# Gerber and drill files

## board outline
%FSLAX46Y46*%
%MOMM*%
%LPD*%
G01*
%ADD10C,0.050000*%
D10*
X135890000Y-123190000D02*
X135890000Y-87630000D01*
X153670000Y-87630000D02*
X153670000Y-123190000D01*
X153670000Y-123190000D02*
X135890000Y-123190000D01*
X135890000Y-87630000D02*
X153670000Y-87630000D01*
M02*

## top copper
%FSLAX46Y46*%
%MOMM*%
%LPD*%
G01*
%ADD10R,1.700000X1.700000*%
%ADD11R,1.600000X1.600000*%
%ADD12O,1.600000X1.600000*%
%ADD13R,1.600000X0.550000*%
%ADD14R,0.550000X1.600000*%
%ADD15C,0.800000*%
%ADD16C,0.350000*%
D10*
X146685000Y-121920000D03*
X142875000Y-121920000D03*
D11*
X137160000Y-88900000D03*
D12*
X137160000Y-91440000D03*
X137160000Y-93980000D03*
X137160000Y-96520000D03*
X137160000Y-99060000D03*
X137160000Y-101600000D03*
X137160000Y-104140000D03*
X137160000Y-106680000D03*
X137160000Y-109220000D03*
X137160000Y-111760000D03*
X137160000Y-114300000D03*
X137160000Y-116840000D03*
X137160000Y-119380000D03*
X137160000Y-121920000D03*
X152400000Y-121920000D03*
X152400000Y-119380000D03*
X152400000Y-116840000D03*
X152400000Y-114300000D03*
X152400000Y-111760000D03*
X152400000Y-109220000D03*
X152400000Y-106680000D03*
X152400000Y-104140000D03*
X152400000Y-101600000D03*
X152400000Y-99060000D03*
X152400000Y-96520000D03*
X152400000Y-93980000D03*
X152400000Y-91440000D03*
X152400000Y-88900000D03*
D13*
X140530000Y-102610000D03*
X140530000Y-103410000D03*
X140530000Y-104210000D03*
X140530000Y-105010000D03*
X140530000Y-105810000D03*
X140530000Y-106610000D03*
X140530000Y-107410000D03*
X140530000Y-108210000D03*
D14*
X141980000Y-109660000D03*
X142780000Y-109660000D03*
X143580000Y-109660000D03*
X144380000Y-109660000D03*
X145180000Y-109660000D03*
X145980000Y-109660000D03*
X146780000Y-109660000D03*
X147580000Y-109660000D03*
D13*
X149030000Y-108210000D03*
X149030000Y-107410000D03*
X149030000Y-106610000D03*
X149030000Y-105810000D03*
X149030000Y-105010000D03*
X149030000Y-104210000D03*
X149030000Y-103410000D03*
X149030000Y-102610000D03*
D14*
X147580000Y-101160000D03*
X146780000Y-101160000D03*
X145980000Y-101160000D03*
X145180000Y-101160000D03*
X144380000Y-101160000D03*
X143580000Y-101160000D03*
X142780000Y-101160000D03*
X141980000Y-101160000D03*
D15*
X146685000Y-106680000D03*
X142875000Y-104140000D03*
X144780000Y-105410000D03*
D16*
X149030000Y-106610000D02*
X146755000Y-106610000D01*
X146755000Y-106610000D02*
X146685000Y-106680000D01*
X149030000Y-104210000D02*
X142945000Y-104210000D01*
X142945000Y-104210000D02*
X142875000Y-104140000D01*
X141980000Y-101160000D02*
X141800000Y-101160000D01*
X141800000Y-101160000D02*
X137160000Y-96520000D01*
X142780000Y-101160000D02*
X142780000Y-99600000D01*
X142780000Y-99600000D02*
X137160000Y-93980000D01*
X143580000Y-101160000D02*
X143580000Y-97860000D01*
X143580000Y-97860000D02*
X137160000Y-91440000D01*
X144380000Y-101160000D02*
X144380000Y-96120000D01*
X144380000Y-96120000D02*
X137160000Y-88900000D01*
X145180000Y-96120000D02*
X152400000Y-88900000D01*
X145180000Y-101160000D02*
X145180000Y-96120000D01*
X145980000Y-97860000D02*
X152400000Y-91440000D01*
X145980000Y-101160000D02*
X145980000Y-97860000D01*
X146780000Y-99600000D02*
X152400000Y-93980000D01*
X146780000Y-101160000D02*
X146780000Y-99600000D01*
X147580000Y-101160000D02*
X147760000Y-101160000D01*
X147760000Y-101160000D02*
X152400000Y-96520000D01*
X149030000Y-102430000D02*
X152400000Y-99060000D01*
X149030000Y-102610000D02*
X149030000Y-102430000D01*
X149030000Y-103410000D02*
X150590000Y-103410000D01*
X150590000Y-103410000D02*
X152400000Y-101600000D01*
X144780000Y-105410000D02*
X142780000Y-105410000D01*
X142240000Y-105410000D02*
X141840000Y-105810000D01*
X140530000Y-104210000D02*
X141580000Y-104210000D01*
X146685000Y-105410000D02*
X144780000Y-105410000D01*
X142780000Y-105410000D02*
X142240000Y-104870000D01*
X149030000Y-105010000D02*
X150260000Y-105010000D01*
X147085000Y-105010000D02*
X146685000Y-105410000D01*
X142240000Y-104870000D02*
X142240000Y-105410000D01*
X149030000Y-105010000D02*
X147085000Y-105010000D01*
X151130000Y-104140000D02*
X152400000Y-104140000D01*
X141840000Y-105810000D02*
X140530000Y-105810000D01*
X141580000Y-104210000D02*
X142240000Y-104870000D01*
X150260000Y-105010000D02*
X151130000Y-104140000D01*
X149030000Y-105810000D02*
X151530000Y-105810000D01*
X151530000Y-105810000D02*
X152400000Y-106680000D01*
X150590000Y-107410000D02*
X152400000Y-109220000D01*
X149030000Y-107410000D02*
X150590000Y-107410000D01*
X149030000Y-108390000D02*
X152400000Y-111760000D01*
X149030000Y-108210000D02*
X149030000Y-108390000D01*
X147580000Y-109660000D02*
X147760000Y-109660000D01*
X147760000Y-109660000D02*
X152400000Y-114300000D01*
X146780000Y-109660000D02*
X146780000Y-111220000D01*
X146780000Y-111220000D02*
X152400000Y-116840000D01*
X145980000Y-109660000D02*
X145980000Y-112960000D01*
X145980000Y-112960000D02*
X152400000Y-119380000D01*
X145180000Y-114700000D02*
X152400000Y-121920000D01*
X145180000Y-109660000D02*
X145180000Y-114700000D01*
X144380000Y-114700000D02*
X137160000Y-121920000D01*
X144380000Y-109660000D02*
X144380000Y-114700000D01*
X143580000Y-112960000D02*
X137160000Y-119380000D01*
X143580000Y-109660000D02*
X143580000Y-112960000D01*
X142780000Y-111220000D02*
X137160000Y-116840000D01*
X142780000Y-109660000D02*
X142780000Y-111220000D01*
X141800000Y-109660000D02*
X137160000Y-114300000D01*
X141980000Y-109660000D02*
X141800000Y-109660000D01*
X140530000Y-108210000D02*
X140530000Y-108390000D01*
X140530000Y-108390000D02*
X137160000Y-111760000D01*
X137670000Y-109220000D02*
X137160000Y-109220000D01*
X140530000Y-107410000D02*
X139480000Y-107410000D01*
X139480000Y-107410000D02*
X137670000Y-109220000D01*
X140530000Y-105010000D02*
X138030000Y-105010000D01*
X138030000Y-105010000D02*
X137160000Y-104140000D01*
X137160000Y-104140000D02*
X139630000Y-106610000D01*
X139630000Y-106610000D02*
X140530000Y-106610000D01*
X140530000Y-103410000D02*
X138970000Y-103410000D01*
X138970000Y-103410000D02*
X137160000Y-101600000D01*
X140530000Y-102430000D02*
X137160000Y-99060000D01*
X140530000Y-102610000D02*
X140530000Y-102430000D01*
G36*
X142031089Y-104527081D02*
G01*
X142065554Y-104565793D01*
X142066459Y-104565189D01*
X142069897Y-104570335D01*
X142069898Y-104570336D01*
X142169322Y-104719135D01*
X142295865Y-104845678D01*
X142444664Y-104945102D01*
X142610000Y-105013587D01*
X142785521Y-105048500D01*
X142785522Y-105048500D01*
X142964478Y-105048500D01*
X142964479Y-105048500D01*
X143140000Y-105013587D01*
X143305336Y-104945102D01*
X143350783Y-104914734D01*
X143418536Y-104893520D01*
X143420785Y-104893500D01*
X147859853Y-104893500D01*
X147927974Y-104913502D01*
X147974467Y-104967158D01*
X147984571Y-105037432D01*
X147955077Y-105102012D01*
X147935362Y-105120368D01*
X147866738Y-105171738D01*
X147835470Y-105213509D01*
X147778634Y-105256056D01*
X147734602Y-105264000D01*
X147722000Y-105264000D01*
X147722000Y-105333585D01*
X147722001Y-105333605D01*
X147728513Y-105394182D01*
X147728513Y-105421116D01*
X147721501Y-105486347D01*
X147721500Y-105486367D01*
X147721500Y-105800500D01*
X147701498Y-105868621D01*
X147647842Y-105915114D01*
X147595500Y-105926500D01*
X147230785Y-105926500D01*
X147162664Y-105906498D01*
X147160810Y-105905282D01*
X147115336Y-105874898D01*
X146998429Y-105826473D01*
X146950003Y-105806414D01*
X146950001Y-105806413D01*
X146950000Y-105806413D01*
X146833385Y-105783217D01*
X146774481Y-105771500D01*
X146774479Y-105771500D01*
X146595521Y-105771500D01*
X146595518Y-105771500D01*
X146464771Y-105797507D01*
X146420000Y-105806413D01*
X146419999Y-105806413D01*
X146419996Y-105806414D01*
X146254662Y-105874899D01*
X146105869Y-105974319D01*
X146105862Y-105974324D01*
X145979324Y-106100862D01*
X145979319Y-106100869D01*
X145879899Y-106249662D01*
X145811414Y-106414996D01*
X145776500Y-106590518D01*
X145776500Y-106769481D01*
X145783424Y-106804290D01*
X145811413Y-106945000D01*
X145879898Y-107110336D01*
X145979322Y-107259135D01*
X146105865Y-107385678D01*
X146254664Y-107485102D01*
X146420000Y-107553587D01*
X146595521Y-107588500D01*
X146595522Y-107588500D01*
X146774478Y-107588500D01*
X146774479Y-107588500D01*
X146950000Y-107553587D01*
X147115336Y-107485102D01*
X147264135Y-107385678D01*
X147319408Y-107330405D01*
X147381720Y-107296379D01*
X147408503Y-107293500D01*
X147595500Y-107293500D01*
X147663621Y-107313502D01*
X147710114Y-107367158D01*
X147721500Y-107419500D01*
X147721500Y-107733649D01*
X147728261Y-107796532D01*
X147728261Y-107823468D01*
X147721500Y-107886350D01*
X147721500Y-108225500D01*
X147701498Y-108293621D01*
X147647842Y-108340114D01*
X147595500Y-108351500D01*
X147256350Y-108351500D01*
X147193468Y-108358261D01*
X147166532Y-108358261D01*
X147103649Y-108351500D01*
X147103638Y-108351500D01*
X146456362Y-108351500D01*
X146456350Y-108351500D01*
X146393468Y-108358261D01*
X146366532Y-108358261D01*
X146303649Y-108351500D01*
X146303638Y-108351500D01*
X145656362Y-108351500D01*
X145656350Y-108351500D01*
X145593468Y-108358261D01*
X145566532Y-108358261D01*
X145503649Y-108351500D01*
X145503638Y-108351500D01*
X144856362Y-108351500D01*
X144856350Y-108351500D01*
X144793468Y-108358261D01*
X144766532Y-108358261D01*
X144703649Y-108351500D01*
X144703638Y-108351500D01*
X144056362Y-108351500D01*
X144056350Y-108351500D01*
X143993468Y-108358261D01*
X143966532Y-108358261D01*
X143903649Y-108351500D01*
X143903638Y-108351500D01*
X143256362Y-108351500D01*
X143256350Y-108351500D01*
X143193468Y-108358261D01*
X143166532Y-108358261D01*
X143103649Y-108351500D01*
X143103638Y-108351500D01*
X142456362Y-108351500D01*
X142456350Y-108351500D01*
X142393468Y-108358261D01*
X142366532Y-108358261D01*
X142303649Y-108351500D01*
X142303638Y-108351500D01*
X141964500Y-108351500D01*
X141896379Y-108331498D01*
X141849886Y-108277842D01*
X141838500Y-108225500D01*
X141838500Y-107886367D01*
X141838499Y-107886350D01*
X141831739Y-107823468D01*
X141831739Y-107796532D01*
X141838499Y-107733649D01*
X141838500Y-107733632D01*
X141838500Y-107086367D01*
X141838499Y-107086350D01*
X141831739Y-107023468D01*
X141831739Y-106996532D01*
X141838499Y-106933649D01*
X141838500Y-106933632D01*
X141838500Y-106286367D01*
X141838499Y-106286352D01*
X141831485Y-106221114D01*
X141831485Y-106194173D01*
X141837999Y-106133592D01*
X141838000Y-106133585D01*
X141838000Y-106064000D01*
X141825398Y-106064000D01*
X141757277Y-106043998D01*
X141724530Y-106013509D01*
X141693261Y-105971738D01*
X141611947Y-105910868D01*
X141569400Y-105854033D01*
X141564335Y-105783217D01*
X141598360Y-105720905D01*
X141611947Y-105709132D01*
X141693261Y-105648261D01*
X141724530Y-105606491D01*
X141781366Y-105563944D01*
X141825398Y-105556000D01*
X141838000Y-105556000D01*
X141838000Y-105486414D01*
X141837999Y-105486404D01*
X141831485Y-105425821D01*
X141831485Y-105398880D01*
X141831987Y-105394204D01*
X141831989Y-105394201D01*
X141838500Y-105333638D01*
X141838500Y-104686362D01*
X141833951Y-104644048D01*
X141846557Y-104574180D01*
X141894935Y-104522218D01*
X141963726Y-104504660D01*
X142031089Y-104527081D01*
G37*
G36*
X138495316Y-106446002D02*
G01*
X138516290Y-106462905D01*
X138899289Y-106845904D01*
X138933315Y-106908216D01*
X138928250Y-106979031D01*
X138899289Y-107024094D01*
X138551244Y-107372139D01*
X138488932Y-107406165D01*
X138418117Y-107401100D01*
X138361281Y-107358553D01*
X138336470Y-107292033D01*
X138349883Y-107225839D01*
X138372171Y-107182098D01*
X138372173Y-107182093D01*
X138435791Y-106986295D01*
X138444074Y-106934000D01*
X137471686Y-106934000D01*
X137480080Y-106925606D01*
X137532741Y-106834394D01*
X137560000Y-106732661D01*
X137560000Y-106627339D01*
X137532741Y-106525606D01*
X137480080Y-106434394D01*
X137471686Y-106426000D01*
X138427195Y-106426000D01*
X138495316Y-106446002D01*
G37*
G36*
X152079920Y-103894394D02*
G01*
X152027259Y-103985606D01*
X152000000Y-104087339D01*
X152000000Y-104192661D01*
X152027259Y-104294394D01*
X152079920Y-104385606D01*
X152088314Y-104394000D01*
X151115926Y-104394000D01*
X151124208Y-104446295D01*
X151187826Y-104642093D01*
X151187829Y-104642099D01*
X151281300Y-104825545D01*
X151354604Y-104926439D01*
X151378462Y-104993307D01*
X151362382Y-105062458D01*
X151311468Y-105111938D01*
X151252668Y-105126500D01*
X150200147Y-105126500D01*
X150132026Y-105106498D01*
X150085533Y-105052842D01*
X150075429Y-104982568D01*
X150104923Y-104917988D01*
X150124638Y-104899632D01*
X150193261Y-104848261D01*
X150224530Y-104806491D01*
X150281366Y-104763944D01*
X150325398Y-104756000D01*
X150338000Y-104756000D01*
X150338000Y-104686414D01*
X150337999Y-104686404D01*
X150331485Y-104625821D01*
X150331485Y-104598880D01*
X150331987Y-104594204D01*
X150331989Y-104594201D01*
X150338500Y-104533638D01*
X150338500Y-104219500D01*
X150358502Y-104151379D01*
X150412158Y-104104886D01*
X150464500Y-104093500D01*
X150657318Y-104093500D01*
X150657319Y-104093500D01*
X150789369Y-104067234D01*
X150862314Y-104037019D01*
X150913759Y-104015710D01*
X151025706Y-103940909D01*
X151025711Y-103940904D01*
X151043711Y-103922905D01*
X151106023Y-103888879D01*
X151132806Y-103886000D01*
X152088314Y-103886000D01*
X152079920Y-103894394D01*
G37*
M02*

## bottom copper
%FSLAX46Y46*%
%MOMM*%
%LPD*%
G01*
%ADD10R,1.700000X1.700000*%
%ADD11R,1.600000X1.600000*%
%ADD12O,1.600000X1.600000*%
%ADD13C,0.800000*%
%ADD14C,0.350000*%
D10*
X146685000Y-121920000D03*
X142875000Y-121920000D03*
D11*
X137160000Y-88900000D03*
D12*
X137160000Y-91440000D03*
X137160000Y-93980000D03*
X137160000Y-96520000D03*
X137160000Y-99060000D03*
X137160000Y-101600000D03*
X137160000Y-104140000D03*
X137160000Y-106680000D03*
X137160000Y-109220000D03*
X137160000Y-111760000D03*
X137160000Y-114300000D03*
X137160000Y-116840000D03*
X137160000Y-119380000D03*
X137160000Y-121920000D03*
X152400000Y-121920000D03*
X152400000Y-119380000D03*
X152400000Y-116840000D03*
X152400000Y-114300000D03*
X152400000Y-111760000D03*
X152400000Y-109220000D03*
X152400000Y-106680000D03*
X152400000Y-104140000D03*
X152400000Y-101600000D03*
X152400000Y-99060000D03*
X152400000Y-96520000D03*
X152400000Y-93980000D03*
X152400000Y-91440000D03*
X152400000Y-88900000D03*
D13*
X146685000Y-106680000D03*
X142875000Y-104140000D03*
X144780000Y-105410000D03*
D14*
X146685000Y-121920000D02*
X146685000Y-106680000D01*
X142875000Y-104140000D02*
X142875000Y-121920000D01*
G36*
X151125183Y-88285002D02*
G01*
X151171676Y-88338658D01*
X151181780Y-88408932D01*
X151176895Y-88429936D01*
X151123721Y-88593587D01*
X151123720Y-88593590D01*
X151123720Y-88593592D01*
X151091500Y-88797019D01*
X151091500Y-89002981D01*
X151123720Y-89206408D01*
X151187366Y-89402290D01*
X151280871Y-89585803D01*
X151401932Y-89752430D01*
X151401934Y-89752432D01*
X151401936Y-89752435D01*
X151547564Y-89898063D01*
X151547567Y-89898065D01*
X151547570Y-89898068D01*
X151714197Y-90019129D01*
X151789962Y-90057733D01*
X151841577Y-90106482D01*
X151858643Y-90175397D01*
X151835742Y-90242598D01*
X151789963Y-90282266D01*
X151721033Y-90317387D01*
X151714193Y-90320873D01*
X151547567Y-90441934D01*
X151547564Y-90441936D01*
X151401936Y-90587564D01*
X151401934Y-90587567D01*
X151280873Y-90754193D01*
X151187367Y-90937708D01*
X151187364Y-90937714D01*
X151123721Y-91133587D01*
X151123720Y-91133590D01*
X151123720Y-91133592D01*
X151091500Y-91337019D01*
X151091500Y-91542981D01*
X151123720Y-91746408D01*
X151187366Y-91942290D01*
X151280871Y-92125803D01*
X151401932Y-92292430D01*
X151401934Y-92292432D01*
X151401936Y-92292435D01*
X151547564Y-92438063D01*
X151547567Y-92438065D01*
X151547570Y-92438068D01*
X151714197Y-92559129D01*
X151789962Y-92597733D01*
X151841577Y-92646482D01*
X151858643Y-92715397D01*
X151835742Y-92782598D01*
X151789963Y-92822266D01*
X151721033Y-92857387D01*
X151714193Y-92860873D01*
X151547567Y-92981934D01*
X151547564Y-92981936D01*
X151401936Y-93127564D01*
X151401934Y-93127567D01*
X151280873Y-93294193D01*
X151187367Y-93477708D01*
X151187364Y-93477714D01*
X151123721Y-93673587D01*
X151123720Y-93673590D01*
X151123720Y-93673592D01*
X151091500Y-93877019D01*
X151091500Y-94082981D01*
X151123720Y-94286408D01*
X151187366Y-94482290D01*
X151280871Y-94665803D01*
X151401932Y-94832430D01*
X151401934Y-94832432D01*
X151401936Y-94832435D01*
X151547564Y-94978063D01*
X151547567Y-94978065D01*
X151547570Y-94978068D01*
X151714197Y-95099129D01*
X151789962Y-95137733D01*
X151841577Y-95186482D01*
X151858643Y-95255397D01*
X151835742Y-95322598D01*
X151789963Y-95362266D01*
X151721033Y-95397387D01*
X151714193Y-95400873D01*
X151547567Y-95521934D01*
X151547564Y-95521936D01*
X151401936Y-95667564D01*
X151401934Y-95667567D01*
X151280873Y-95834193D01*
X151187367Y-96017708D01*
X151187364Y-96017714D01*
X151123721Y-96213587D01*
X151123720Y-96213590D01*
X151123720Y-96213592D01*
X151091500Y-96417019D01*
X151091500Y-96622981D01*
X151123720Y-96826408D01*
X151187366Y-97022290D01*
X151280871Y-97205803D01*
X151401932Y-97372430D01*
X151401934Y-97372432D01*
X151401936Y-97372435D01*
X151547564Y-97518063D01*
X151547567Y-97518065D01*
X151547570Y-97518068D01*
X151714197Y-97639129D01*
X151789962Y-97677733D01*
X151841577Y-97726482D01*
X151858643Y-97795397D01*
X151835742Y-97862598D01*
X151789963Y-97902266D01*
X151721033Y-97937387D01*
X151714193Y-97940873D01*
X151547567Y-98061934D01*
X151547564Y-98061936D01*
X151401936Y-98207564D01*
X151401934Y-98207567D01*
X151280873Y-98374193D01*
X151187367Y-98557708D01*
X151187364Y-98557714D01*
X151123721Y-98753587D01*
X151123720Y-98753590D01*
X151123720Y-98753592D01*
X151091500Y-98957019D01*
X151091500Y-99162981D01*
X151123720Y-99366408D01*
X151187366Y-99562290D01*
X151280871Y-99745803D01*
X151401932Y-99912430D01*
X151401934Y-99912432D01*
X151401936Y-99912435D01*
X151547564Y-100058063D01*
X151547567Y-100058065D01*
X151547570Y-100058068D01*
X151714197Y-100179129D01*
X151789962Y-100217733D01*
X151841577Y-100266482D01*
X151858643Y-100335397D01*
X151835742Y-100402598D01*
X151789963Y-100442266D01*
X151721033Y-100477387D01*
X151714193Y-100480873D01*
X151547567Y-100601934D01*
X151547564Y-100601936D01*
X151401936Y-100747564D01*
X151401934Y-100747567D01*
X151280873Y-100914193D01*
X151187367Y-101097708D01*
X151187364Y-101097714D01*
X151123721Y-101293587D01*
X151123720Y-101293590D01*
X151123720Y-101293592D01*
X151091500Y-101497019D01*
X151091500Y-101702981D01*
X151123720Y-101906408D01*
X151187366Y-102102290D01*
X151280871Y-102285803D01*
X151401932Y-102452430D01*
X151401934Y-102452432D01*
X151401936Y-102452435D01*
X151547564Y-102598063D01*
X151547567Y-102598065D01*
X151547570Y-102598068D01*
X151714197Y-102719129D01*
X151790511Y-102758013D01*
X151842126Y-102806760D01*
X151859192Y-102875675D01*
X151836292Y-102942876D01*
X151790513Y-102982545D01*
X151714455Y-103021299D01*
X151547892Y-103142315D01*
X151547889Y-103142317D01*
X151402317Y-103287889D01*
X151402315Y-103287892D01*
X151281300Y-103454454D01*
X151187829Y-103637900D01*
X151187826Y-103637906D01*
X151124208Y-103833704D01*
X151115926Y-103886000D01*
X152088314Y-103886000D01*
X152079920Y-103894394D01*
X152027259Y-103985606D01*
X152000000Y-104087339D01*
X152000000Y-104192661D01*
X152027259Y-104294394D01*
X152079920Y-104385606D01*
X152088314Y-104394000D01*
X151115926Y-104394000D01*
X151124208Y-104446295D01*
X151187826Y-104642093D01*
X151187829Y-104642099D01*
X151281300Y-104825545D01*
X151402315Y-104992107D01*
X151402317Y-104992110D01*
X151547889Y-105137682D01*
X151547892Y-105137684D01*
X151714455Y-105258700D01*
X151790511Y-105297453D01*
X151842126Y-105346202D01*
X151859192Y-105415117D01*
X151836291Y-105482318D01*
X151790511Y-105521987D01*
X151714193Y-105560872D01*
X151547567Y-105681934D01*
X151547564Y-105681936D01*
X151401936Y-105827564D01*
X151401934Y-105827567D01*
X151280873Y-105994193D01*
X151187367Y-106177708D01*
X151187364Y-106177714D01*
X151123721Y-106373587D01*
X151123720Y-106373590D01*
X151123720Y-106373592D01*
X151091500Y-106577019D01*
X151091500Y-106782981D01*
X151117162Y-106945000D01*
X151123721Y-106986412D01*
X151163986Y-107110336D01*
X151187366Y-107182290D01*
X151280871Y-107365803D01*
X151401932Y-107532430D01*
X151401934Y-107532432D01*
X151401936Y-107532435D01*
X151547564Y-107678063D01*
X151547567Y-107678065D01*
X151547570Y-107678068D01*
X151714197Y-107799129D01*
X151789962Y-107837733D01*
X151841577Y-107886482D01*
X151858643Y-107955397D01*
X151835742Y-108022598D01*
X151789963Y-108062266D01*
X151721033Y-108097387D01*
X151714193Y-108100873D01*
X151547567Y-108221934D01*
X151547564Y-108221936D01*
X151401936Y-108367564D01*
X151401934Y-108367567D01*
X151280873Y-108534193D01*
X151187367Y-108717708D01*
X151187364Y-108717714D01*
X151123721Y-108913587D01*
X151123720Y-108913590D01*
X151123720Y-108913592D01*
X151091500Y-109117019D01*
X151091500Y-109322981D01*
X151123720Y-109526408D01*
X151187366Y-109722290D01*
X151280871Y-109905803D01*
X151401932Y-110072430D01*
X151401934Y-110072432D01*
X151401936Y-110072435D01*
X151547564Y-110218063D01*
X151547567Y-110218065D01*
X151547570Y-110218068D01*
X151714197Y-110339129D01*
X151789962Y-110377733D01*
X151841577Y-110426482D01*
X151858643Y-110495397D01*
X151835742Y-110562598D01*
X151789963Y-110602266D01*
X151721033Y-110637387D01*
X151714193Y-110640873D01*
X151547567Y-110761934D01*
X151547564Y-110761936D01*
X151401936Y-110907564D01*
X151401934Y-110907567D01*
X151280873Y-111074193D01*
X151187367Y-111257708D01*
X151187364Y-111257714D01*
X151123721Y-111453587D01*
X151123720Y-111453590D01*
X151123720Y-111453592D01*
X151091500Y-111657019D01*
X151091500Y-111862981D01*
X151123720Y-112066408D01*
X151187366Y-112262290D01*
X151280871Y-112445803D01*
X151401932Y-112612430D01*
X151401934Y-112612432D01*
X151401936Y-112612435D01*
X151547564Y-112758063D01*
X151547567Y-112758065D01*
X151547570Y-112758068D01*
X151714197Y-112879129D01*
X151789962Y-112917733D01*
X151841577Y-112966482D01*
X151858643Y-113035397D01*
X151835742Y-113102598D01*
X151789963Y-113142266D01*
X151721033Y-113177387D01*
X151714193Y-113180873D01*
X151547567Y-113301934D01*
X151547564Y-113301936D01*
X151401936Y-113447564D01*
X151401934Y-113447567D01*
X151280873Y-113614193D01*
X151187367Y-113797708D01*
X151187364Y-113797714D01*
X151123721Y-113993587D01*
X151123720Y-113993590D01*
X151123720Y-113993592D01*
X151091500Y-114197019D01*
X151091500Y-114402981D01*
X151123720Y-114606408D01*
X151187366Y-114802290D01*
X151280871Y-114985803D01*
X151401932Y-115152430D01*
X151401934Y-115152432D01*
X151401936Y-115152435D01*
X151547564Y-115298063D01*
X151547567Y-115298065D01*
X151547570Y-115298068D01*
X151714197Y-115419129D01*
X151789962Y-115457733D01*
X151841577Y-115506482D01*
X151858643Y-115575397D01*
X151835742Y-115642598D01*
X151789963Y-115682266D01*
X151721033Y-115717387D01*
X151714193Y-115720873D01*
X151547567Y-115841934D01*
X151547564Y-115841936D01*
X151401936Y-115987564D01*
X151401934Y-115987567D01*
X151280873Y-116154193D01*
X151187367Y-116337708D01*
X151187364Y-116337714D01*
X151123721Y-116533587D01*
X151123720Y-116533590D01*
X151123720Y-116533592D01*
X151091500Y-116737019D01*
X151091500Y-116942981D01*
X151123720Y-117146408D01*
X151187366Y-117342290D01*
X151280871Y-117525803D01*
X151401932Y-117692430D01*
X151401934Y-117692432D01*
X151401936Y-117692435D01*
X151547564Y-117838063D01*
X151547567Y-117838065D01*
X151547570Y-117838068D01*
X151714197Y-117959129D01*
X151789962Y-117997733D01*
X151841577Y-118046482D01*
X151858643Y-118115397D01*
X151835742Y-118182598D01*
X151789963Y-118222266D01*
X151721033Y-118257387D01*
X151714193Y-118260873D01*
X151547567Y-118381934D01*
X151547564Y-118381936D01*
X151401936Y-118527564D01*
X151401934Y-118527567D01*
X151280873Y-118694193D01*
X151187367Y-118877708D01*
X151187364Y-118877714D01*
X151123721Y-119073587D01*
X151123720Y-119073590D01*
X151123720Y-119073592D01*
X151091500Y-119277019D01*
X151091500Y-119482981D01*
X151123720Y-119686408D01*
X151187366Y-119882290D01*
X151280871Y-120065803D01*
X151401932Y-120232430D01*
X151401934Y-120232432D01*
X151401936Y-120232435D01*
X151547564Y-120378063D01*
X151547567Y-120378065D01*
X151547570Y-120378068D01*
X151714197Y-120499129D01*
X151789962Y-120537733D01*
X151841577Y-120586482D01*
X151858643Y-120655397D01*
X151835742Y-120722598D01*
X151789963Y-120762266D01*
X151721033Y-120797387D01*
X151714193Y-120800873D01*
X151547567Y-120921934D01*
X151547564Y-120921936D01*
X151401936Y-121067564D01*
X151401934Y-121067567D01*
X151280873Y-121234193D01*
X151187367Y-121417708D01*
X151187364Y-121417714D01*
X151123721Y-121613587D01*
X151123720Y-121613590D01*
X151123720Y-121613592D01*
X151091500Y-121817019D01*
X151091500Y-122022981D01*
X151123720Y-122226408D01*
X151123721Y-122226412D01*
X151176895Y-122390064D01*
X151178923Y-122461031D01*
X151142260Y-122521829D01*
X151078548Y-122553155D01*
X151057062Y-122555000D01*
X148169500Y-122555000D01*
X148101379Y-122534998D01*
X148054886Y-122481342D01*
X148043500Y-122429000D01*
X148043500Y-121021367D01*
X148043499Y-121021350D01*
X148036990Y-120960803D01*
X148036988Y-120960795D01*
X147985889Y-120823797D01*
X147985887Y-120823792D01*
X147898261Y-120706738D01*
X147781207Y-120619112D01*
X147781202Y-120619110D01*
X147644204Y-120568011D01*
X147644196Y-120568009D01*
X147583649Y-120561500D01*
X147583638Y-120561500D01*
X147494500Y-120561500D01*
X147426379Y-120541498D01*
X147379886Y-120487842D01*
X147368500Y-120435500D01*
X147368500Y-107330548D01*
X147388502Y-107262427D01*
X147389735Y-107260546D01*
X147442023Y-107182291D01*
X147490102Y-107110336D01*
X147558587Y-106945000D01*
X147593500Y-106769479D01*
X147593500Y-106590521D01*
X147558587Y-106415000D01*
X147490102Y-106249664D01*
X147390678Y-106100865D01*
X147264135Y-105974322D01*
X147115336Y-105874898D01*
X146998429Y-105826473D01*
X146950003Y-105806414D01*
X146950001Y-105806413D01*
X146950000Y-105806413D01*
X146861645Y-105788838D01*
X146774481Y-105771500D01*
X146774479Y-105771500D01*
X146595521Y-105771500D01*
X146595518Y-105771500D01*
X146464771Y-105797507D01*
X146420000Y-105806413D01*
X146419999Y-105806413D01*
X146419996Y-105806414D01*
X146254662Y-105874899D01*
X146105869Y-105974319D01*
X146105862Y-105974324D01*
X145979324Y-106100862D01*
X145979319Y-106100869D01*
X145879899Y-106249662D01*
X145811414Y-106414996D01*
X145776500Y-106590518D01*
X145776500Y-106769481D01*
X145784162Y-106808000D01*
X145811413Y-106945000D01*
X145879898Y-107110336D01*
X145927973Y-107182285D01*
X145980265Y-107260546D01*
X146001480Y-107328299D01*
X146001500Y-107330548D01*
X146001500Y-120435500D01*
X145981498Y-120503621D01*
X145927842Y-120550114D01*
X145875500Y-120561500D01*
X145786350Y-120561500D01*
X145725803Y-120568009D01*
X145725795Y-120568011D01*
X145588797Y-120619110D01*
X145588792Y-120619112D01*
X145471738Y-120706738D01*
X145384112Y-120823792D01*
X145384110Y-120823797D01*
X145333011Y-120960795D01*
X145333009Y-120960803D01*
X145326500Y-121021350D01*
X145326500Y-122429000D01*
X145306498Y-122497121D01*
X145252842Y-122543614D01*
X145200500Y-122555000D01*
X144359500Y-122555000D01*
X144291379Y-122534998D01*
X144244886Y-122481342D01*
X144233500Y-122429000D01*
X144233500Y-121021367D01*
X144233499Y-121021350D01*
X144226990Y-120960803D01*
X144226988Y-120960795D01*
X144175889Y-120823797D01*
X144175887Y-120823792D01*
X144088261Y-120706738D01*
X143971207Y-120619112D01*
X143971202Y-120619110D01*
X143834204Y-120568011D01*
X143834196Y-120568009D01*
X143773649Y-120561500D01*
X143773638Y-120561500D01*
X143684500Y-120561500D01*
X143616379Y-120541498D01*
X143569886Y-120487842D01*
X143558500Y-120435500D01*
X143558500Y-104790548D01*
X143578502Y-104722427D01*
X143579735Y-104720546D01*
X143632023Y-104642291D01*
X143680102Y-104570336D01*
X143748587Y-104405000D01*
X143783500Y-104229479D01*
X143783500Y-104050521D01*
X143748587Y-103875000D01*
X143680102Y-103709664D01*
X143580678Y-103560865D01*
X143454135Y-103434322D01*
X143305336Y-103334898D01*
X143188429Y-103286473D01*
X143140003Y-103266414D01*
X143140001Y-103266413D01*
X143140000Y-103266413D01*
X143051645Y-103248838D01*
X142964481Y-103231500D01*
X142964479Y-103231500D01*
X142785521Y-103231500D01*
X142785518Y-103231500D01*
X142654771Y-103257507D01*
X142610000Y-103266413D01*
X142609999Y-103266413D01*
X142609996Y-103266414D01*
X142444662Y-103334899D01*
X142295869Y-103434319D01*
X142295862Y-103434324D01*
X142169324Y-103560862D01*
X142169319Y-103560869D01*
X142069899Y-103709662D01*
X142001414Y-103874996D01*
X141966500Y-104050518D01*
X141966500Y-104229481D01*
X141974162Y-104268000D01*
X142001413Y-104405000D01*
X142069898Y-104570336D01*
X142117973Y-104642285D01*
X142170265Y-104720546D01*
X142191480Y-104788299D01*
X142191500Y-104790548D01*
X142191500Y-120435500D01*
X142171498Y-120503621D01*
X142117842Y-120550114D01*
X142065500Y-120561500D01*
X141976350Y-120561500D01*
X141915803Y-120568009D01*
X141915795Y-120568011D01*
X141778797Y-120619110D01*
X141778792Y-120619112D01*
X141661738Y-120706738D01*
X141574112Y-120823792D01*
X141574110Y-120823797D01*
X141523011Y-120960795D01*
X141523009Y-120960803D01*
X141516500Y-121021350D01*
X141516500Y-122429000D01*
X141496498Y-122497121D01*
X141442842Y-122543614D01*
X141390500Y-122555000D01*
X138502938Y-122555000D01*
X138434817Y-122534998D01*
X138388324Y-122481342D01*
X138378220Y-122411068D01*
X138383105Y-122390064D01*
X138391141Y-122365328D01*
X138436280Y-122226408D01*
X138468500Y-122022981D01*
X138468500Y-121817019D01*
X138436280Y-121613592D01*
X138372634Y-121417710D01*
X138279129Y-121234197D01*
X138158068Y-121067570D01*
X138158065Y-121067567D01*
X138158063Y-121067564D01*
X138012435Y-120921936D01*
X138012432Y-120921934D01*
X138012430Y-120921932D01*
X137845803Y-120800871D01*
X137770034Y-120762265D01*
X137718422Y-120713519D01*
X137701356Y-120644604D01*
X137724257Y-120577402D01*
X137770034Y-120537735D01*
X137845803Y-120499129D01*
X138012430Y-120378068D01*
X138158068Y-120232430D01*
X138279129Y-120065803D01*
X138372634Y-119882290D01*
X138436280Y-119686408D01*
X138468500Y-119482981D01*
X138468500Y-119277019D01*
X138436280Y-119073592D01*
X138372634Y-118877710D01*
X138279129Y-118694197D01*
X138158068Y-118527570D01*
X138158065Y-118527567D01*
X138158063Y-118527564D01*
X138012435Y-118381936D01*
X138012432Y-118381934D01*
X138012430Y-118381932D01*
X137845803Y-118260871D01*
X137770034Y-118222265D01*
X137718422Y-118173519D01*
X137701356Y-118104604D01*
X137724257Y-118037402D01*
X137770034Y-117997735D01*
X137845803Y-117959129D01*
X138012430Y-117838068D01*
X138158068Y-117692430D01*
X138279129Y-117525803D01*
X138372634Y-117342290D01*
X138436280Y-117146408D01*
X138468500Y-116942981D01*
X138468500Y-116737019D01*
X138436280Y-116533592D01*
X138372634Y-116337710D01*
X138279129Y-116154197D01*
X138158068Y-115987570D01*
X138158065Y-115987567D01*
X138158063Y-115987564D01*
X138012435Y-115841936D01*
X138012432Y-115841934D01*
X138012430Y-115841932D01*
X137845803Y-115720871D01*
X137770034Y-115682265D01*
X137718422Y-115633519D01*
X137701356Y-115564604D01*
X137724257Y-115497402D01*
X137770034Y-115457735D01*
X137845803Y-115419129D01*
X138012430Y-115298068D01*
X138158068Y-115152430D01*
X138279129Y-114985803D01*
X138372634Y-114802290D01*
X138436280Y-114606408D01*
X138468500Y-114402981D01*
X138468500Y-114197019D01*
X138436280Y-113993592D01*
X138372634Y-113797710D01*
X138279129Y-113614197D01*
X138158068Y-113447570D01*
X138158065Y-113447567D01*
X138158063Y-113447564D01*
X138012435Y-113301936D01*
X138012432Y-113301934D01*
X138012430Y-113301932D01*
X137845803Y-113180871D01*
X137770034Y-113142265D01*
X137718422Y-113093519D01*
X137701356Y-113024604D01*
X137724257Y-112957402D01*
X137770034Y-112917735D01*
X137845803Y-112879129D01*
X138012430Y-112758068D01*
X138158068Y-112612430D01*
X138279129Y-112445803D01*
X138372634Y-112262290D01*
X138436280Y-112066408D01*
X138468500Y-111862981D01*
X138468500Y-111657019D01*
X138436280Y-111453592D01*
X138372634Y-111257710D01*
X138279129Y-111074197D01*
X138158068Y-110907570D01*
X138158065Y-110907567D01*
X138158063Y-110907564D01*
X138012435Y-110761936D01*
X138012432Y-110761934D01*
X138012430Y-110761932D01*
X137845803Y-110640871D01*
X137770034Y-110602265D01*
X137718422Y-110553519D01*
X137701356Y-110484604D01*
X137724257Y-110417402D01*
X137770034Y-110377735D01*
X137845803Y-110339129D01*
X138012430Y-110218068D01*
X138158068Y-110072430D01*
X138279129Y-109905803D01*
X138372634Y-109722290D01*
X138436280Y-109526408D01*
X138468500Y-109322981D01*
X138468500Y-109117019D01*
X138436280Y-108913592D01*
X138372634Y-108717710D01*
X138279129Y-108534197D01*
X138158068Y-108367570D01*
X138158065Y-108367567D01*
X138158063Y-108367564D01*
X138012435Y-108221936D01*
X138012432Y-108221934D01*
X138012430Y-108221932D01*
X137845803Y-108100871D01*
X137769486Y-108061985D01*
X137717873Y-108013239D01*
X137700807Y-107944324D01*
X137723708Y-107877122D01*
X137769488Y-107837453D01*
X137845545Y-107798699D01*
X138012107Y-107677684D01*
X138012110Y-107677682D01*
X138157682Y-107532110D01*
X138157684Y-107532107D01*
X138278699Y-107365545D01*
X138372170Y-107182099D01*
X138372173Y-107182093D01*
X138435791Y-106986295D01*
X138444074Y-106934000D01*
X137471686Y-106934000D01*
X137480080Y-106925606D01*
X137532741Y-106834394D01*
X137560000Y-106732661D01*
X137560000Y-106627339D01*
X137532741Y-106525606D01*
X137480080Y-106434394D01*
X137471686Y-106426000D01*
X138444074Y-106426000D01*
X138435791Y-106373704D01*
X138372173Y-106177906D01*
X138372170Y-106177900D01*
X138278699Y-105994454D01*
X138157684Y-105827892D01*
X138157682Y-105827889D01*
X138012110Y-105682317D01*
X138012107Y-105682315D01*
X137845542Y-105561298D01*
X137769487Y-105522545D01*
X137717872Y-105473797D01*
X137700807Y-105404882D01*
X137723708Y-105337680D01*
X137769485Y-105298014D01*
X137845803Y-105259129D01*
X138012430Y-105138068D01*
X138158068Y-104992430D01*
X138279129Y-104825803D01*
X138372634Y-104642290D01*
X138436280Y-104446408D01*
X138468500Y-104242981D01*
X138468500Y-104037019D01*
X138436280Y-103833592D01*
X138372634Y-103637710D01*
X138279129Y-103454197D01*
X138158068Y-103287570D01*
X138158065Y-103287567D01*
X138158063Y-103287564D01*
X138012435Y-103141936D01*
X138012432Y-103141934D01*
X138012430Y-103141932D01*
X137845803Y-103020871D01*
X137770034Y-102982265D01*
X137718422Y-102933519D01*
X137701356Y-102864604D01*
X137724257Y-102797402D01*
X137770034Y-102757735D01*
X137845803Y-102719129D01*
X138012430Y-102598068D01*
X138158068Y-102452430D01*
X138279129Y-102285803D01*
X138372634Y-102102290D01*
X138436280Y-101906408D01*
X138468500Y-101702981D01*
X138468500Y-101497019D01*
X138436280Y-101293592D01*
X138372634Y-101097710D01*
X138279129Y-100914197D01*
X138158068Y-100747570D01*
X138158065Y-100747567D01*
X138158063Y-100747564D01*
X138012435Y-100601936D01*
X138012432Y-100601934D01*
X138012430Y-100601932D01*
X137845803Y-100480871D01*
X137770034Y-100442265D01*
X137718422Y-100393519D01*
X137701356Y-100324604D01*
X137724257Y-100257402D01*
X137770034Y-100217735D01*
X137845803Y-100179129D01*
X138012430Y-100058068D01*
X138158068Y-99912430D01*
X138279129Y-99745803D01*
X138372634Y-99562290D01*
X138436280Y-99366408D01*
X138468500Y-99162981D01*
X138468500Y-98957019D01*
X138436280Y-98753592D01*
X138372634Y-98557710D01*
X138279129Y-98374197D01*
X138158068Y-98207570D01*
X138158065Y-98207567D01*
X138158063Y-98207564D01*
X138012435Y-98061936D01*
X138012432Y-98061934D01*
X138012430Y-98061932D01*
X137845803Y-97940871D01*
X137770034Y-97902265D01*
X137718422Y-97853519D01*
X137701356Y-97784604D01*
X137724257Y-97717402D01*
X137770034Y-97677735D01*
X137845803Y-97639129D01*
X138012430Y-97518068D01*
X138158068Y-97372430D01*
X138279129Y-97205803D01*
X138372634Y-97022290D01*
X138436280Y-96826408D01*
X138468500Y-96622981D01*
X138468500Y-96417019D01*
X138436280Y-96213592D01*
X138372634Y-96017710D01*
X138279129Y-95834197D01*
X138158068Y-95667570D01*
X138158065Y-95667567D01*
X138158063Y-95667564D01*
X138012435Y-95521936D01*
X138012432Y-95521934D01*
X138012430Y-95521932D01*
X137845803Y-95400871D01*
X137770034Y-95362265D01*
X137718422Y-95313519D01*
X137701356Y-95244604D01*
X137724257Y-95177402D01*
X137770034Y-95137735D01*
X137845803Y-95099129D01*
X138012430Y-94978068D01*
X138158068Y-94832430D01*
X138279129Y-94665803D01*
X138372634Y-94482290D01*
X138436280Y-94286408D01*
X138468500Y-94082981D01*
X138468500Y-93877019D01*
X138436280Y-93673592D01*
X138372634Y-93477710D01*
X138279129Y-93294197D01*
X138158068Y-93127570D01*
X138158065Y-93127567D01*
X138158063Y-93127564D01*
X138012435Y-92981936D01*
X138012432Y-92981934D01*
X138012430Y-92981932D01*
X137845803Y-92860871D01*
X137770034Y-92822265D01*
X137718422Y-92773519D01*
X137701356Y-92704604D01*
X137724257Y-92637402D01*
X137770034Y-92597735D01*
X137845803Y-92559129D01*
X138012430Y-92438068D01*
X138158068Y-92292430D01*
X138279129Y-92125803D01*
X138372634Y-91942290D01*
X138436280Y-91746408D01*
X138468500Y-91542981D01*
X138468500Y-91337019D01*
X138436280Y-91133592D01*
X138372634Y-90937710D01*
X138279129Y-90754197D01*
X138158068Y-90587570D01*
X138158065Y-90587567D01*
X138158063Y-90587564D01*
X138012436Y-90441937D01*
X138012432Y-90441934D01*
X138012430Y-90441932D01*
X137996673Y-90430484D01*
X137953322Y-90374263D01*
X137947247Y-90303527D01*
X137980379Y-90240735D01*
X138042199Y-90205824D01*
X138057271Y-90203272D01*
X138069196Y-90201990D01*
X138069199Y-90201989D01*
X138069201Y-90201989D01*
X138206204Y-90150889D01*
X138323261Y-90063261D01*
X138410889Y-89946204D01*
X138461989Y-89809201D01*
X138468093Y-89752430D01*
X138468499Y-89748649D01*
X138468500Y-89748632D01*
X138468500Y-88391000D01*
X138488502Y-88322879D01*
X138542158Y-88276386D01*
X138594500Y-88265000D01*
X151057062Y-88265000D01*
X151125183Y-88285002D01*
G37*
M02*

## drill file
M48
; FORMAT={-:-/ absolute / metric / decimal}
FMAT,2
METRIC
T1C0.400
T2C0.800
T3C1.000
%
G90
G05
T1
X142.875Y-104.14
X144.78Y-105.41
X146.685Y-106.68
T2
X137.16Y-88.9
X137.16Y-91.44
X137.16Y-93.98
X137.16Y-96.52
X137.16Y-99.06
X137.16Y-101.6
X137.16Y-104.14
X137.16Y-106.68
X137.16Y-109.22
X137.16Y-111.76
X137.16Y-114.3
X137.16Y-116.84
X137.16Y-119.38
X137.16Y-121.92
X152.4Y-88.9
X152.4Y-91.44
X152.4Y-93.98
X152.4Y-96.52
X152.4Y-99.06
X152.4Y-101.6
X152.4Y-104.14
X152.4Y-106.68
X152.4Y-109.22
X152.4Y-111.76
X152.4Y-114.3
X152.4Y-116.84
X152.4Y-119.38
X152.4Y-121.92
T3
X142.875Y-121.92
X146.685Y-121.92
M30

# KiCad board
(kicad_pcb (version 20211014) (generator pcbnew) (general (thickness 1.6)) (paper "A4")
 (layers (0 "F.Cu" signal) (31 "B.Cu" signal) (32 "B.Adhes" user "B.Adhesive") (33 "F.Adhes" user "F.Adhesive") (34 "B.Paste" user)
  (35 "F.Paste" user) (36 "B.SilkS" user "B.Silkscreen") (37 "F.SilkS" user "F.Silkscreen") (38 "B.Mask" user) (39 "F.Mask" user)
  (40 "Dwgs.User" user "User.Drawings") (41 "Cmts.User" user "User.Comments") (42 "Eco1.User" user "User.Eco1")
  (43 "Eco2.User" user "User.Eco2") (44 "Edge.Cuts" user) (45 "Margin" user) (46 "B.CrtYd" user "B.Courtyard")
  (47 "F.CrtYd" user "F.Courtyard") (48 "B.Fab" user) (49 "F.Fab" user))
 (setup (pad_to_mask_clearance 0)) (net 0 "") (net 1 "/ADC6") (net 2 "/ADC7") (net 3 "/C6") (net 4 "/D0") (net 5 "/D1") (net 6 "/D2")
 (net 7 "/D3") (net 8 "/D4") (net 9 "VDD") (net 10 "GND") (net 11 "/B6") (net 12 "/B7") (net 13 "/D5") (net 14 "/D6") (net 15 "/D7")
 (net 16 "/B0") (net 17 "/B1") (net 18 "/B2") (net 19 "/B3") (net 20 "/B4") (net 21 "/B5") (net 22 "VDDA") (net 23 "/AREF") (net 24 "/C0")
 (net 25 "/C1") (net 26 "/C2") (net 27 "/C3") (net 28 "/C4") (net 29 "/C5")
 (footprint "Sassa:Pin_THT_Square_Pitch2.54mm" (layer "F.Cu") (at 146.685 121.92)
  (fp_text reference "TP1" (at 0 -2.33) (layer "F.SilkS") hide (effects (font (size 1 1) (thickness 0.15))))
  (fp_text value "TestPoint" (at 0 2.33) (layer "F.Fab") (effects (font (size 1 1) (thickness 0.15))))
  (pad "1" thru_hole rect locked (at 0 0) (size 1.7 1.7) (drill 1) (layers *.Cu *.Mask) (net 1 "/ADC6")))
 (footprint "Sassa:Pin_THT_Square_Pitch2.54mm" (layer "F.Cu") (at 142.875 121.92)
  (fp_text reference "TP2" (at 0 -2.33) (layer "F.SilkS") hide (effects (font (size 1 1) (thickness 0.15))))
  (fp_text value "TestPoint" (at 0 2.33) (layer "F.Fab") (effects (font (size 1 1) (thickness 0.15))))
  (pad "1" thru_hole rect locked (at 0 0) (size 1.7 1.7) (drill 1) (layers *.Cu *.Mask) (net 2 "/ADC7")))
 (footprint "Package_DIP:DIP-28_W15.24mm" (layer "F.Cu") (at 137.16 88.9)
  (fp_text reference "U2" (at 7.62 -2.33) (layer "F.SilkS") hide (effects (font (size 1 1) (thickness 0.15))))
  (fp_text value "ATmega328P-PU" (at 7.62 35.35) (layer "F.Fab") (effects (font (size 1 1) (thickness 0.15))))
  (pad "1" thru_hole rect (at 0 0) (size 1.6 1.6) (drill 0.8) (layers *.Cu *.Mask) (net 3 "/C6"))
  (pad "2" thru_hole oval (at 0 2.54) (size 1.6 1.6) (drill 0.8) (layers *.Cu *.Mask) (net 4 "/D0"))
  (pad "3" thru_hole oval (at 0 5.08) (size 1.6 1.6) (drill 0.8) (layers *.Cu *.Mask) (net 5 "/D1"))
  (pad "4" thru_hole oval (at 0 7.62) (size 1.6 1.6) (drill 0.8) (layers *.Cu *.Mask) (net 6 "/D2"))
  (pad "5" thru_hole oval (at 0 10.16) (size 1.6 1.6) (drill 0.8) (layers *.Cu *.Mask) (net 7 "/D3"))
  (pad "6" thru_hole oval (at 0 12.7) (size 1.6 1.6) (drill 0.8) (layers *.Cu *.Mask) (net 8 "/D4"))
  (pad "7" thru_hole oval (at 0 15.24) (size 1.6 1.6) (drill 0.8) (layers *.Cu *.Mask) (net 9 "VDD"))
  (pad "8" thru_hole oval (at 0 17.78) (size 1.6 1.6) (drill 0.8) (layers *.Cu *.Mask) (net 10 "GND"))
  (pad "9" thru_hole oval (at 0 20.32) (size 1.6 1.6) (drill 0.8) (layers *.Cu *.Mask) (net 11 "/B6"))
  (pad "10" thru_hole oval (at 0 22.86) (size 1.6 1.6) (drill 0.8) (layers *.Cu *.Mask) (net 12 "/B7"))
  (pad "11" thru_hole oval (at 0 25.4) (size 1.6 1.6) (drill 0.8) (layers *.Cu *.Mask) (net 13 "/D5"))
  (pad "12" thru_hole oval (at 0 27.94) (size 1.6 1.6) (drill 0.8) (layers *.Cu *.Mask) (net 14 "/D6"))
  (pad "13" thru_hole oval (at 0 30.48) (size 1.6 1.6) (drill 0.8) (layers *.Cu *.Mask) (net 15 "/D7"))
  (pad "14" thru_hole oval (at 0 33.02) (size 1.6 1.6) (drill 0.8) (layers *.Cu *.Mask) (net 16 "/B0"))
  (pad "15" thru_hole oval (at 15.24 33.02) (size 1.6 1.6) (drill 0.8) (layers *.Cu *.Mask) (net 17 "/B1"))
  (pad "16" thru_hole oval (at 15.24 30.48) (size 1.6 1.6) (drill 0.8) (layers *.Cu *.Mask) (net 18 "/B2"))
  (pad "17" thru_hole oval (at 15.24 27.94) (size 1.6 1.6) (drill 0.8) (layers *.Cu *.Mask) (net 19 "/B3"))
  (pad "18" thru_hole oval (at 15.24 25.4) (size 1.6 1.6) (drill 0.8) (layers *.Cu *.Mask) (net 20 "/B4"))
  (pad "19" thru_hole oval (at 15.24 22.86) (size 1.6 1.6) (drill 0.8) (layers *.Cu *.Mask) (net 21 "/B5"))
  (pad "20" thru_hole oval (at 15.24 20.32) (size 1.6 1.6) (drill 0.8) (layers *.Cu *.Mask) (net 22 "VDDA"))
  (pad "21" thru_hole oval (at 15.24 17.78) (size 1.6 1.6) (drill 0.8) (layers *.Cu *.Mask) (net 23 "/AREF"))
  (pad "22" thru_hole oval (at 15.24 15.24) (size 1.6 1.6) (drill 0.8) (layers *.Cu *.Mask) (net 10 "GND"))
  (pad "23" thru_hole oval (at 15.24 12.7) (size 1.6 1.6) (drill 0.8) (layers *.Cu *.Mask) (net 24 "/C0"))
  (pad "24" thru_hole oval (at 15.24 10.16) (size 1.6 1.6) (drill 0.8) (layers *.Cu *.Mask) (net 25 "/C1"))
  (pad "25" thru_hole oval (at 15.24 7.62) (size 1.6 1.6) (drill 0.8) (layers *.Cu *.Mask) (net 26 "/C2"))
  (pad "26" thru_hole oval (at 15.24 5.08) (size 1.6 1.6) (drill 0.8) (layers *.Cu *.Mask) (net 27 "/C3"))
  (pad "27" thru_hole oval (at 15.24 2.54) (size 1.6 1.6) (drill 0.8) (layers *.Cu *.Mask) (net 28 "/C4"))
  (pad "28" thru_hole oval (at 15.24 0) (size 1.6 1.6) (drill 0.8) (layers *.Cu *.Mask) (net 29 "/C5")))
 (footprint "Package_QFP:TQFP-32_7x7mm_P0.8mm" (layer "F.Cu") (at 144.78 105.41)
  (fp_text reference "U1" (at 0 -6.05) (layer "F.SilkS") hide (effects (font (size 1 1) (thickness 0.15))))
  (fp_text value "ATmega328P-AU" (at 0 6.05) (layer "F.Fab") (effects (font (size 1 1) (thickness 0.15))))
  (pad "1" smd rect (at -4.25 -2.8) (size 1.6 0.55) (layers "F.Cu" "F.Paste" "F.Mask") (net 7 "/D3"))
  (pad "2" smd rect (at -4.25 -2) (size 1.6 0.55) (layers "F.Cu" "F.Paste" "F.Mask") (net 8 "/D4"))
  (pad "3" smd rect (at -4.25 -1.2) (size 1.6 0.55) (layers "F.Cu" "F.Paste" "F.Mask") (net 10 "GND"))
  (pad "4" smd rect (at -4.25 -0.4) (size 1.6 0.55) (layers "F.Cu" "F.Paste" "F.Mask") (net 9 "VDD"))
  (pad "5" smd rect (at -4.25 0.4) (size 1.6 0.55) (layers "F.Cu" "F.Paste" "F.Mask") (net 10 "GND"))
  (pad "6" smd rect (at -4.25 1.2) (size 1.6 0.55) (layers "F.Cu" "F.Paste" "F.Mask") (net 9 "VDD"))
  (pad "7" smd rect (at -4.25 2) (size 1.6 0.55) (layers "F.Cu" "F.Paste" "F.Mask") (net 11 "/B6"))
  (pad "8" smd rect (at -4.25 2.8) (size 1.6 0.55) (layers "F.Cu" "F.Paste" "F.Mask") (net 12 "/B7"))
  (pad "9" smd rect (at -2.8 4.25 90) (size 1.6 0.55) (layers "F.Cu" "F.Paste" "F.Mask") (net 13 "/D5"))
  (pad "10" smd rect (at -2 4.25 90) (size 1.6 0.55) (layers "F.Cu" "F.Paste" "F.Mask") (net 14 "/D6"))
  (pad "11" smd rect (at -1.2 4.25 90) (size 1.6 0.55) (layers "F.Cu" "F.Paste" "F.Mask") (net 15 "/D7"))
  (pad "12" smd rect (at -0.4 4.25 90) (size 1.6 0.55) (layers "F.Cu" "F.Paste" "F.Mask") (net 16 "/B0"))
  (pad "13" smd rect (at 0.4 4.25 90) (size 1.6 0.55) (layers "F.Cu" "F.Paste" "F.Mask") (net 17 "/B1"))
  (pad "14" smd rect (at 1.2 4.25 90) (size 1.6 0.55) (layers "F.Cu" "F.Paste" "F.Mask") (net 18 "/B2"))
  (pad "15" smd rect (at 2 4.25 90) (size 1.6 0.55) (layers "F.Cu" "F.Paste" "F.Mask") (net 19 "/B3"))
  (pad "16" smd rect (at 2.8 4.25 90) (size 1.6 0.55) (layers "F.Cu" "F.Paste" "F.Mask") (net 20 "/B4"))
  (pad "17" smd rect (at 4.25 2.8) (size 1.6 0.55) (layers "F.Cu" "F.Paste" "F.Mask") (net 21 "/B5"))
  (pad "18" smd rect (at 4.25 2) (size 1.6 0.55) (layers "F.Cu" "F.Paste" "F.Mask") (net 22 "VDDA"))
  (pad "19" smd rect (at 4.25 1.2) (size 1.6 0.55) (layers "F.Cu" "F.Paste" "F.Mask") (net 1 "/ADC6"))
  (pad "20" smd rect (at 4.25 0.4) (size 1.6 0.55) (layers "F.Cu" "F.Paste" "F.Mask") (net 23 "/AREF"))
  (pad "21" smd rect (at 4.25 -0.4) (size 1.6 0.55) (layers "F.Cu" "F.Paste" "F.Mask") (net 10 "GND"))
  (pad "22" smd rect (at 4.25 -1.2) (size 1.6 0.55) (layers "F.Cu" "F.Paste" "F.Mask") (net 2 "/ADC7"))
  (pad "23" smd rect (at 4.25 -2) (size 1.6 0.55) (layers "F.Cu" "F.Paste" "F.Mask") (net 24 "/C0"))
  (pad "24" smd rect (at 4.25 -2.8) (size 1.6 0.55) (layers "F.Cu" "F.Paste" "F.Mask") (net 25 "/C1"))
  (pad "25" smd rect (at 2.8 -4.25 90) (size 1.6 0.55) (layers "F.Cu" "F.Paste" "F.Mask") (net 26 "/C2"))
  (pad "26" smd rect (at 2 -4.25 90) (size 1.6 0.55) (layers "F.Cu" "F.Paste" "F.Mask") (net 27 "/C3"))
  (pad "27" smd rect (at 1.2 -4.25 90) (size 1.6 0.55) (layers "F.Cu" "F.Paste" "F.Mask") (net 28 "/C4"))
  (pad "28" smd rect (at 0.4 -4.25 90) (size 1.6 0.55) (layers "F.Cu" "F.Paste" "F.Mask") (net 29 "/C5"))
  (pad "29" smd rect (at -0.4 -4.25 90) (size 1.6 0.55) (layers "F.Cu" "F.Paste" "F.Mask") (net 3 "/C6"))
  (pad "30" smd rect (at -1.2 -4.25 90) (size 1.6 0.55) (layers "F.Cu" "F.Paste" "F.Mask") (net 4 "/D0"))
  (pad "31" smd rect (at -2 -4.25 90) (size 1.6 0.55) (layers "F.Cu" "F.Paste" "F.Mask") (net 5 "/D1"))
  (pad "32" smd rect (at -2.8 -4.25 90) (size 1.6 0.55) (layers "F.Cu" "F.Paste" "F.Mask") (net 6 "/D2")))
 (gr_line (start 135.89 123.19) (end 135.89 87.63) (layer "Edge.Cuts") (width 0.05))
 (gr_line (start 153.67 87.63) (end 153.67 123.19) (layer "Edge.Cuts") (width 0.05))
 (gr_line (start 153.67 123.19) (end 135.89 123.19) (layer "Edge.Cuts") (width 0.05))
 (gr_line (start 135.89 87.63) (end 153.67 87.63) (layer "Edge.Cuts") (width 0.05))
 (segment (start 149.03 106.61) (end 146.755 106.61) (width 0.35) (layer "F.Cu") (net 1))
 (segment (start 146.755 106.61) (end 146.685 106.68) (width 0.35) (layer "F.Cu") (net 1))
 (via (at 146.685 106.68) (size 0.8) (drill 0.4) (layers "F.Cu" "B.Cu") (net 1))
 (segment (start 146.685 121.92) (end 146.685 106.68) (width 0.35) (layer "B.Cu") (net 1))
 (segment (start 149.03 104.21) (end 142.945 104.21) (width 0.35) (layer "F.Cu") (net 2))
 (segment (start 142.945 104.21) (end 142.875 104.14) (width 0.35) (layer "F.Cu") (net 2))
 (via (at 142.875 104.14) (size 0.8) (drill 0.4) (layers "F.Cu" "B.Cu") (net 2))
 (segment (start 142.875 104.14) (end 142.875 121.92) (width 0.35) (layer "B.Cu") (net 2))
 (segment (start 141.98 101.16) (end 141.8 101.16) (width 0.35) (layer "F.Cu") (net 6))
 (segment (start 141.8 101.16) (end 137.16 96.52) (width 0.35) (layer "F.Cu") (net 6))
 (segment (start 142.78 101.16) (end 142.78 99.6) (width 0.35) (layer "F.Cu") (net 5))
 (segment (start 142.78 99.6) (end 137.16 93.98) (width 0.35) (layer "F.Cu") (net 5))
 (segment (start 143.58 101.16) (end 143.58 97.86) (width 0.35) (layer "F.Cu") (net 4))
 (segment (start 143.58 97.86) (end 137.16 91.44) (width 0.35) (layer "F.Cu") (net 4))
 (segment (start 144.38 101.16) (end 144.38 96.12) (width 0.35) (layer "F.Cu") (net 3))
 (segment (start 144.38 96.12) (end 137.16 88.9) (width 0.35) (layer "F.Cu") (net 3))
 (segment (start 145.18 96.12) (end 152.4 88.9) (width 0.35) (layer "F.Cu") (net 29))
 (segment (start 145.18 101.16) (end 145.18 96.12) (width 0.35) (layer "F.Cu") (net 29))
 (segment (start 145.98 97.86) (end 152.4 91.44) (width 0.35) (layer "F.Cu") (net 28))
 (segment (start 145.98 101.16) (end 145.98 97.86) (width 0.35) (layer "F.Cu") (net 28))
 (segment (start 146.78 99.6) (end 152.4 93.98) (width 0.35) (layer "F.Cu") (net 27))
 (segment (start 146.78 101.16) (end 146.78 99.6) (width 0.35) (layer "F.Cu") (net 27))
 (segment (start 147.58 101.16) (end 147.76 101.16) (width 0.35) (layer "F.Cu") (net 26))
 (segment (start 147.76 101.16) (end 152.4 96.52) (width 0.35) (layer "F.Cu") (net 26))
 (segment (start 149.03 102.43) (end 152.4 99.06) (width 0.35) (layer "F.Cu") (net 25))
 (segment (start 149.03 102.61) (end 149.03 102.43) (width 0.35) (layer "F.Cu") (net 25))
 (segment (start 149.03 103.41) (end 150.59 103.41) (width 0.35) (layer "F.Cu") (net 24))
 (segment (start 150.59 103.41) (end 152.4 101.6) (width 0.35) (layer "F.Cu") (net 24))
 (segment (start 144.78 105.41) (end 142.78 105.41) (width 0.35) (layer "F.Cu") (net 10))
 (segment (start 142.24 105.41) (end 141.84 105.81) (width 0.35) (layer "F.Cu") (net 10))
 (segment (start 140.53 104.21) (end 141.58 104.21) (width 0.35) (layer "F.Cu") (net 10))
 (segment (start 146.685 105.41) (end 144.78 105.41) (width 0.35) (layer "F.Cu") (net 10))
 (segment (start 142.78 105.41) (end 142.24 104.87) (width 0.35) (layer "F.Cu") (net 10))
 (segment (start 149.03 105.01) (end 150.26 105.01) (width 0.35) (layer "F.Cu") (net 10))
 (segment (start 147.085 105.01) (end 146.685 105.41) (width 0.35) (layer "F.Cu") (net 10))
 (segment (start 142.24 104.87) (end 142.24 105.41) (width 0.35) (layer "F.Cu") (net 10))
 (segment (start 149.03 105.01) (end 147.085 105.01) (width 0.35) (layer "F.Cu") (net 10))
 (segment (start 151.13 104.14) (end 152.4 104.14) (width 0.35) (layer "F.Cu") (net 10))
 (segment (start 141.84 105.81) (end 140.53 105.81) (width 0.35) (layer "F.Cu") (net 10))
 (segment (start 141.58 104.21) (end 142.24 104.87) (width 0.35) (layer "F.Cu") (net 10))
 (segment (start 150.26 105.01) (end 151.13 104.14) (width 0.35) (layer "F.Cu") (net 10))
 (via (at 144.78 105.41) (size 0.8) (drill 0.4) (layers "F.Cu" "B.Cu") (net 10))
 (segment (start 149.03 105.81) (end 151.53 105.81) (width 0.35) (layer "F.Cu") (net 23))
 (segment (start 151.53 105.81) (end 152.4 106.68) (width 0.35) (layer "F.Cu") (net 23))
 (segment (start 150.59 107.41) (end 152.4 109.22) (width 0.35) (layer "F.Cu") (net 22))
 (segment (start 149.03 107.41) (end 150.59 107.41) (width 0.35) (layer "F.Cu") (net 22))
 (segment (start 149.03 108.39) (end 152.4 111.76) (width 0.35) (layer "F.Cu") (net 21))
 (segment (start 149.03 108.21) (end 149.03 108.39) (width 0.35) (layer "F.Cu") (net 21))
 (segment (start 147.58 109.66) (end 147.76 109.66) (width 0.35) (layer "F.Cu") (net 20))
 (segment (start 147.76 109.66) (end 152.4 114.3) (width 0.35) (layer "F.Cu") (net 20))
 (segment (start 146.78 109.66) (end 146.78 111.22) (width 0.35) (layer "F.Cu") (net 19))
 (segment (start 146.78 111.22) (end 152.4 116.84) (width 0.35) (layer "F.Cu") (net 19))
 (segment (start 145.98 109.66) (end 145.98 112.96) (width 0.35) (layer "F.Cu") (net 18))
 (segment (start 145.98 112.96) (end 152.4 119.38) (width 0.35) (layer "F.Cu") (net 18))
 (segment (start 145.18 114.7) (end 152.4 121.92) (width 0.35) (layer "F.Cu") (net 17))
 (segment (start 145.18 109.66) (end 145.18 114.7) (width 0.35) (layer "F.Cu") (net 17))
 (segment (start 144.38 114.7) (end 137.16 121.92) (width 0.35) (layer "F.Cu") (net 16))
 (segment (start 144.38 109.66) (end 144.38 114.7) (width 0.35) (layer "F.Cu") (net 16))
 (segment (start 143.58 112.96) (end 137.16 119.38) (width 0.35) (layer "F.Cu") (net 15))
 (segment (start 143.58 109.66) (end 143.58 112.96) (width 0.35) (layer "F.Cu") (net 15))
 (segment (start 142.78 111.22) (end 137.16 116.84) (width 0.35) (layer "F.Cu") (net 14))
 (segment (start 142.78 109.66) (end 142.78 111.22) (width 0.35) (layer "F.Cu") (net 14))
 (segment (start 141.8 109.66) (end 137.16 114.3) (width 0.35) (layer "F.Cu") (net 13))
 (segment (start 141.98 109.66) (end 141.8 109.66) (width 0.35) (layer "F.Cu") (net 13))
 (segment (start 140.53 108.21) (end 140.53 108.39) (width 0.35) (layer "F.Cu") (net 12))
 (segment (start 140.53 108.39) (end 137.16 111.76) (width 0.35) (layer "F.Cu") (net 12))
 (segment (start 137.67 109.22) (end 137.16 109.22) (width 0.35) (layer "F.Cu") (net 11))
 (segment (start 140.53 107.41) (end 139.48 107.41) (width 0.35) (layer "F.Cu") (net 11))
 (segment (start 139.48 107.41) (end 137.67 109.22) (width 0.35) (layer "F.Cu") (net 11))
 (segment (start 140.53 105.01) (end 138.03 105.01) (width 0.35) (layer "F.Cu") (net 9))
 (segment (start 138.03 105.01) (end 137.16 104.14) (width 0.35) (layer "F.Cu") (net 9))
 (segment (start 137.16 104.14) (end 139.63 106.61) (width 0.35) (layer "F.Cu") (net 9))
 (segment (start 139.63 106.61) (end 140.53 106.61) (width 0.35) (layer "F.Cu") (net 9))
 (segment (start 140.53 103.41) (end 138.97 103.41) (width 0.35) (layer "F.Cu") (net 8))
 (segment (start 138.97 103.41) (end 137.16 101.6) (width 0.35) (layer "F.Cu") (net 8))
 (segment (start 140.53 102.43) (end 137.16 99.06) (width 0.35) (layer "F.Cu") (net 7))
 (segment (start 140.53 102.61) (end 140.53 102.43) (width 0.35) (layer "F.Cu") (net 7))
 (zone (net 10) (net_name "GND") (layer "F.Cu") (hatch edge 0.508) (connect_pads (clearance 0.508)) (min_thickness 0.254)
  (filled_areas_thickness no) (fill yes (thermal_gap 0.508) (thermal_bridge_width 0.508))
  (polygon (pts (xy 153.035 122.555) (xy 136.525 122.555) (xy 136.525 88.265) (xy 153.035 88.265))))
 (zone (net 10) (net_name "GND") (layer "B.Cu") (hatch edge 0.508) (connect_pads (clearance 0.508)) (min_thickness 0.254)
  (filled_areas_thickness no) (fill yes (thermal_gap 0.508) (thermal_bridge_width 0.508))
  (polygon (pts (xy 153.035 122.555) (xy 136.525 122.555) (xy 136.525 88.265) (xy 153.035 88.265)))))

